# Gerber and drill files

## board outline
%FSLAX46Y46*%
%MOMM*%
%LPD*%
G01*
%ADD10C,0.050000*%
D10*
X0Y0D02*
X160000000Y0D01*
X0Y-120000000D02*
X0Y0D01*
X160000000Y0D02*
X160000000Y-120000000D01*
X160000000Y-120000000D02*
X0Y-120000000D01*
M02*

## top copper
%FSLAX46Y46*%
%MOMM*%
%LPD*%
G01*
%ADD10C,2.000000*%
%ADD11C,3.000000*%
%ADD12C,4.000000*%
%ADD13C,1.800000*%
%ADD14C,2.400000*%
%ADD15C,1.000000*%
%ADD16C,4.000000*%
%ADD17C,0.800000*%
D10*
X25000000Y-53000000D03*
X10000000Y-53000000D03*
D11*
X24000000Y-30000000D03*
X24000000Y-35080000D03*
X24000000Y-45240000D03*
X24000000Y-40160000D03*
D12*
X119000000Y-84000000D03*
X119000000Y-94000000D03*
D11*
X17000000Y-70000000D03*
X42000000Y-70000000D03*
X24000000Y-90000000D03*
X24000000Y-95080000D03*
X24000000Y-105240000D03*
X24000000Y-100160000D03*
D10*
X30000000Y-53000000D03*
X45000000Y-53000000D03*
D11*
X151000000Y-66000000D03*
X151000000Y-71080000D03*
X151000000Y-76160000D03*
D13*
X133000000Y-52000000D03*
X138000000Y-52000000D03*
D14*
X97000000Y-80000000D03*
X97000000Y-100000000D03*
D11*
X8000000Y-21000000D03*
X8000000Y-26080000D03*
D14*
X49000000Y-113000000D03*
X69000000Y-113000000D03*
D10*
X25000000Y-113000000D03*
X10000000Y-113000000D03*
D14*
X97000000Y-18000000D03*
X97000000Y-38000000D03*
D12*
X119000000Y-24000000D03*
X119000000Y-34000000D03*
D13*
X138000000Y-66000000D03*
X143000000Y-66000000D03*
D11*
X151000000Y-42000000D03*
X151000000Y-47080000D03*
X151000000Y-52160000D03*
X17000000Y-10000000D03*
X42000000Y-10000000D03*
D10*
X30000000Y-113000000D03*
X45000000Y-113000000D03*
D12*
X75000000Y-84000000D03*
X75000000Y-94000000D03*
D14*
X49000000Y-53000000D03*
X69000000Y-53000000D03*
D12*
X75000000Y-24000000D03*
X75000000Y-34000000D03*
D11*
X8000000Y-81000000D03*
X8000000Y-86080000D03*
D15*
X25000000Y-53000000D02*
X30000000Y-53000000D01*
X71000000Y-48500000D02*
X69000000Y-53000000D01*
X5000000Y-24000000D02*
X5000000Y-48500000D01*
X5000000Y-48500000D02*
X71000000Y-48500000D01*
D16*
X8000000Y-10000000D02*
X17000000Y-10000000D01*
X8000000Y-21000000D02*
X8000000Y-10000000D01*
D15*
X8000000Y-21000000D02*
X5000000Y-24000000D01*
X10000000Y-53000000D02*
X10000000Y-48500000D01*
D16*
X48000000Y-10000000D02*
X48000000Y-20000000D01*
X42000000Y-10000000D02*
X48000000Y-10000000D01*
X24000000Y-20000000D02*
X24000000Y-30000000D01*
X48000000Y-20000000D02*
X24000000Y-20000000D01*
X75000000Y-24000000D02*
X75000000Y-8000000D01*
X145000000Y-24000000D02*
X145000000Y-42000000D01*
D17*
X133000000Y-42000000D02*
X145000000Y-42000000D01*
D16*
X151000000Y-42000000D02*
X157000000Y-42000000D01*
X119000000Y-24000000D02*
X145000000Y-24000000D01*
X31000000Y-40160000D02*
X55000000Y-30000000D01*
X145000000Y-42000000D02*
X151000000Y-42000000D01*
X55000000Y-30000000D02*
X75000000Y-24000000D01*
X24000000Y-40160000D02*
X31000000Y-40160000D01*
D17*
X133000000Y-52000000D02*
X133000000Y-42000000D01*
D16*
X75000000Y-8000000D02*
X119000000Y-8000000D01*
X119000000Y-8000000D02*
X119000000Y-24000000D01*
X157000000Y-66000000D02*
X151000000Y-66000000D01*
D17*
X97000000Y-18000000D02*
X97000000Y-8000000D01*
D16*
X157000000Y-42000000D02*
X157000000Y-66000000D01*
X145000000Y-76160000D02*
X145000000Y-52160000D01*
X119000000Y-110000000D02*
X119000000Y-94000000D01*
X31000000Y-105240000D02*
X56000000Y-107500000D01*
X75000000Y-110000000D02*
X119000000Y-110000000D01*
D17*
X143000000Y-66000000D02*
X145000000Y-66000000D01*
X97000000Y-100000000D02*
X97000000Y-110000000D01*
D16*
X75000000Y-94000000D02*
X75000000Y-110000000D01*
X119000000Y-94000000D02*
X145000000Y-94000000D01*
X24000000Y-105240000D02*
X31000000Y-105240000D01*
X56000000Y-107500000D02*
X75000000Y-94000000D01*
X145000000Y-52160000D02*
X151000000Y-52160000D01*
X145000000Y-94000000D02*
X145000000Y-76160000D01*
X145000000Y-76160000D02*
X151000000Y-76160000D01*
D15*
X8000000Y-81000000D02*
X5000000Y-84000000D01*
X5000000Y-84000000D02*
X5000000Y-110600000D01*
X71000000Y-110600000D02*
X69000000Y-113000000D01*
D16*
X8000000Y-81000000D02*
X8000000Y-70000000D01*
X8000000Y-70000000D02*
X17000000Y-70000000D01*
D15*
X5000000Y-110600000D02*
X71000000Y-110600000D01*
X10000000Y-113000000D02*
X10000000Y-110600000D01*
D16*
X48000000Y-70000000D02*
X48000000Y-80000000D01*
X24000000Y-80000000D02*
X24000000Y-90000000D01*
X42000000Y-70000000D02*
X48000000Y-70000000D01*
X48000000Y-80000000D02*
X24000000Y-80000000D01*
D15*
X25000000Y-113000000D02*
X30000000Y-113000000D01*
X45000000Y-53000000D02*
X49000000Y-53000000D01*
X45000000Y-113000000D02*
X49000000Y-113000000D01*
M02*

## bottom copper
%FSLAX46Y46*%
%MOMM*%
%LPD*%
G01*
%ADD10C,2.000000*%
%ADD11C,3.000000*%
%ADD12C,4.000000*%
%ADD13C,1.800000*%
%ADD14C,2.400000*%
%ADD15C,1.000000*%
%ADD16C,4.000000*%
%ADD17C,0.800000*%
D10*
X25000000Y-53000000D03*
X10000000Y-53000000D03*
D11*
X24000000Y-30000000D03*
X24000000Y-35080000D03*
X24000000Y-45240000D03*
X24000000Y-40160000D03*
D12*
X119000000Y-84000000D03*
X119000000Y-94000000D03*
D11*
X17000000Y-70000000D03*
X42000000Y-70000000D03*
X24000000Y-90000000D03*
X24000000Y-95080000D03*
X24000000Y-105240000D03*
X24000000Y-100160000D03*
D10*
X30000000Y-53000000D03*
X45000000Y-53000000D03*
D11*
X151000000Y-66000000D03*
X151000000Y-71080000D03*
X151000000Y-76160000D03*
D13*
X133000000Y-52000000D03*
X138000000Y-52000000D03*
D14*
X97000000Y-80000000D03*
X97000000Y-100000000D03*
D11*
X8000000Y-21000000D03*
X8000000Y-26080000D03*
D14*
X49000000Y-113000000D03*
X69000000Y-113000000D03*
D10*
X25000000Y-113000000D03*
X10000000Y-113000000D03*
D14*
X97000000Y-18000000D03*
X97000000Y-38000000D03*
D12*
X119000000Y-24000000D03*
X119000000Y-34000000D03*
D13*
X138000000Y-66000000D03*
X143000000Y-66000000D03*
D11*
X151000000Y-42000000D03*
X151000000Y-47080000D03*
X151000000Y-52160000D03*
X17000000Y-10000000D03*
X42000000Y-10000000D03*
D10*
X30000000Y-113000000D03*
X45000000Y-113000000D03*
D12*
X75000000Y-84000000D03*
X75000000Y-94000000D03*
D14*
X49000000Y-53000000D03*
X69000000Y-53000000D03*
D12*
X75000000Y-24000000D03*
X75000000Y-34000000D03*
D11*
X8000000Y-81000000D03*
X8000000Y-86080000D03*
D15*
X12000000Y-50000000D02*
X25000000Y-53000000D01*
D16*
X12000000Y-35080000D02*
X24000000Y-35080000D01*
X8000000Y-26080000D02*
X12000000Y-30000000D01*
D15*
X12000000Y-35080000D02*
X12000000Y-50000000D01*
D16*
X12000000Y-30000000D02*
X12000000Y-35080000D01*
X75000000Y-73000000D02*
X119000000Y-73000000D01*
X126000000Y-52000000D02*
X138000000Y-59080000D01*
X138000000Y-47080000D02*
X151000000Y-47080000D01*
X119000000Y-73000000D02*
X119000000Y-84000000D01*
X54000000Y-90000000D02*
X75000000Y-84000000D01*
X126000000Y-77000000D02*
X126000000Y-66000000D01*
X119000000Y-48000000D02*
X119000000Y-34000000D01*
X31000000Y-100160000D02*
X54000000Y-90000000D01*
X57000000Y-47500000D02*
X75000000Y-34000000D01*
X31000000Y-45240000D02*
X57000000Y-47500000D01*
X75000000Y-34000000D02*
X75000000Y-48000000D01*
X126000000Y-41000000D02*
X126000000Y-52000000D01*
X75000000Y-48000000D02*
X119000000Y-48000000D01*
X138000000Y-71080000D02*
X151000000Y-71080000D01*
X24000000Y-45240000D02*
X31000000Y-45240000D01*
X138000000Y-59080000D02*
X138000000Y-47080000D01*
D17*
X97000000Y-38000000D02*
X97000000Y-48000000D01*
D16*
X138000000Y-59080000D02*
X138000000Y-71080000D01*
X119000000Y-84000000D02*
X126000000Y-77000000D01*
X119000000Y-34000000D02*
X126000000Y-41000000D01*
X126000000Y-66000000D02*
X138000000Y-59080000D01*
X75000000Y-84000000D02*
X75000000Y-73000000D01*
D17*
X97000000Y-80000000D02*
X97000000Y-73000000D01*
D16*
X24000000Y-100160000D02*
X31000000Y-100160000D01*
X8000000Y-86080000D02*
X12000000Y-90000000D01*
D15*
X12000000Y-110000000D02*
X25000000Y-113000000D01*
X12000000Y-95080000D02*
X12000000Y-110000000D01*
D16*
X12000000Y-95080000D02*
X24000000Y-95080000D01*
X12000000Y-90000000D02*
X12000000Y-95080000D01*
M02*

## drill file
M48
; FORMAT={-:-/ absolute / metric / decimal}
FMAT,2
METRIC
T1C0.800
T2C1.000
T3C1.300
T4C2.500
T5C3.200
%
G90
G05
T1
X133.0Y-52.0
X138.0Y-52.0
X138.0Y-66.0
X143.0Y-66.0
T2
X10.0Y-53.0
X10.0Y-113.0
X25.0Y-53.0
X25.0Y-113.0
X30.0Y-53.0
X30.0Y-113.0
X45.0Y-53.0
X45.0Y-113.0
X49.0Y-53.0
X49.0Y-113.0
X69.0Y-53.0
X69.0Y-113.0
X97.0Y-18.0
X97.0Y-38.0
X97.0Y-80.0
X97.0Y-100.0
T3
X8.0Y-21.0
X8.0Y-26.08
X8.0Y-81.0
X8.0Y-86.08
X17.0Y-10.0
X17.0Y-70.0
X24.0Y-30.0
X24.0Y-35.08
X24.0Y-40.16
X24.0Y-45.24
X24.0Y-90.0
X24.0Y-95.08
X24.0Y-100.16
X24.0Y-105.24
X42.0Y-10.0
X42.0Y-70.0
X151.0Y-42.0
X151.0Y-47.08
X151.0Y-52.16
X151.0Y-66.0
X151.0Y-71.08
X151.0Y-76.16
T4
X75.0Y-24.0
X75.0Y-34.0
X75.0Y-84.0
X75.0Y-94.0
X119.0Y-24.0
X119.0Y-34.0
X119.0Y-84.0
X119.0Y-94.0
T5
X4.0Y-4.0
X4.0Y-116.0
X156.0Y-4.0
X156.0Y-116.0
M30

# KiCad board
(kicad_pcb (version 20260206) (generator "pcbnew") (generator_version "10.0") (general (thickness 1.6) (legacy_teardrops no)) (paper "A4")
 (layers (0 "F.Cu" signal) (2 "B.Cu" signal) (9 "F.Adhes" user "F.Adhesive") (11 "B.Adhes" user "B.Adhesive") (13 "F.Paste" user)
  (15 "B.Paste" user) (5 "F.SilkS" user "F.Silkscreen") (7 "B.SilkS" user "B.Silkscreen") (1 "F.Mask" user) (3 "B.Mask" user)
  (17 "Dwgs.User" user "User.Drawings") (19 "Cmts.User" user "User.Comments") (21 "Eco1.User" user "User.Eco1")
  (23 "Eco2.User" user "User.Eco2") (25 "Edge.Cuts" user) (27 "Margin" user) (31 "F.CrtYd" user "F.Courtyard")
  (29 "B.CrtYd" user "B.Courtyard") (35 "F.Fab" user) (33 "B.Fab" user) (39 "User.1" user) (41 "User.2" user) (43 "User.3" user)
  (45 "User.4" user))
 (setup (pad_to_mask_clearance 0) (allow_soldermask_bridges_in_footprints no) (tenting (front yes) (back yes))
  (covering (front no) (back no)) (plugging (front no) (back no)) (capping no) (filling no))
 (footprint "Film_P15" (layer "F.Cu") (at 25 53 180)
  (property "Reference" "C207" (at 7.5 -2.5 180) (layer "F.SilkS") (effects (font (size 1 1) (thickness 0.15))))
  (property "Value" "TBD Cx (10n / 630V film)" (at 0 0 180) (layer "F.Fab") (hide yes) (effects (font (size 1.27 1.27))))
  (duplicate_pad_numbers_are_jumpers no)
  (pad "1" thru_hole circle (at 0 0 180) (size 2 2) (drill 1) (layers "*.Cu" "*.Mask") (remove_unused_layers no) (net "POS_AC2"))
  (pad "2" thru_hole circle (at 15 0 180) (size 2 2) (drill 1) (layers "*.Cu" "*.Mask") (remove_unused_layers no) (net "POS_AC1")))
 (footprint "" (layer "F.Cu") (at 156 4)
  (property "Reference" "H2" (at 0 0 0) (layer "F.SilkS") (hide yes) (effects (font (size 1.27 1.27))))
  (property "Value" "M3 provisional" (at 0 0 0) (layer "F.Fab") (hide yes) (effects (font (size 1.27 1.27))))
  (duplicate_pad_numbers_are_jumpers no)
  (pad "" np_thru_hole circle (at 0 0) (size 3.2 3.2) (drill 3.2) (layers "*.Cu" "*.Mask")))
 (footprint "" (layer "F.Cu") (at 4 4)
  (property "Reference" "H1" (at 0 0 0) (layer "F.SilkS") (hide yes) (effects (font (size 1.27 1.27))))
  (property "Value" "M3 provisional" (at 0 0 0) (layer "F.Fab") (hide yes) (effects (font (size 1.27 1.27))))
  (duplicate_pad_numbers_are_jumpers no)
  (pad "" np_thru_hole circle (at 0 0) (size 3.2 3.2) (drill 3.2) (layers "*.Cu" "*.Mask")))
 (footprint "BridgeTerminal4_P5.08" (layer "F.Cu") (at 24 30 -90)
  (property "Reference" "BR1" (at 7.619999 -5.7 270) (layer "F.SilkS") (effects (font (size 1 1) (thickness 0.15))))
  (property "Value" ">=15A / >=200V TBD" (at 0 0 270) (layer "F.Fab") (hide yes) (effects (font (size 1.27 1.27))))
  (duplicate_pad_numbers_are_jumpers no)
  (pad "AC1" thru_hole circle (at 0 0 270) (size 3 3) (drill 1.3) (layers "*.Cu" "*.Mask") (remove_unused_layers no) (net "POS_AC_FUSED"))
  (pad "AC2" thru_hole circle (at 5.08 0 270) (size 3 3) (drill 1.3) (layers "*.Cu" "*.Mask") (remove_unused_layers no) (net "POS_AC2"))
  (pad "N" thru_hole circle (at 15.24 0 270) (size 3 3) (drill 1.3) (layers "*.Cu" "*.Mask") (remove_unused_layers no) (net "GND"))
  (pad "P" thru_hole circle (at 10.16 0 270) (size 3 3) (drill 1.3) (layers "*.Cu" "*.Mask") (remove_unused_layers no) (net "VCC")))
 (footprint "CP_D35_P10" (layer "F.Cu") (at 119 84 -90)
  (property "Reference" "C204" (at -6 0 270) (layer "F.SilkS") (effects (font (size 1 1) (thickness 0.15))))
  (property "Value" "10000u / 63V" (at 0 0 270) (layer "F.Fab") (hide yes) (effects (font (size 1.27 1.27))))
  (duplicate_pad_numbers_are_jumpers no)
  (pad "1" thru_hole circle (at 0 0 270) (size 4 4) (drill 2.5) (layers "*.Cu" "*.Mask") (remove_unused_layers no) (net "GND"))
  (pad "2" thru_hole circle (at 10 0 270) (size 4 4) (drill 2.5) (layers "*.Cu" "*.Mask") (remove_unused_layers no) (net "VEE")))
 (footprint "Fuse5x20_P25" (layer "F.Cu") (at 17 70)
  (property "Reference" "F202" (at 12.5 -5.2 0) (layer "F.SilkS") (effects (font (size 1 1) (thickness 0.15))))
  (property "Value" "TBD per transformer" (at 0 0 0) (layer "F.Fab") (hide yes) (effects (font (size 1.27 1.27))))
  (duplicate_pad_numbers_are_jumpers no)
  (pad "1" thru_hole circle (at 0 0) (size 3 3) (drill 1.3) (layers "*.Cu" "*.Mask") (remove_unused_layers no) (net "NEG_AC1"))
  (pad "2" thru_hole circle (at 25 0) (size 3 3) (drill 1.3) (layers "*.Cu" "*.Mask") (remove_unused_layers no) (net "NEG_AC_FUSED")))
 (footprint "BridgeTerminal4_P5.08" (layer "F.Cu") (at 24 90 -90)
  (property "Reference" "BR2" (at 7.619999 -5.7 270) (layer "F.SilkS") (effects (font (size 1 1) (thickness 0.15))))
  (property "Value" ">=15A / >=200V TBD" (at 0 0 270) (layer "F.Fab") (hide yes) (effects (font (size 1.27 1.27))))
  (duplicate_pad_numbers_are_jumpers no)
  (pad "AC1" thru_hole circle (at 0 0 270) (size 3 3) (drill 1.3) (layers "*.Cu" "*.Mask") (remove_unused_layers no) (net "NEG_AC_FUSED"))
  (pad "AC2" thru_hole circle (at 5.08 0 270) (size 3 3) (drill 1.3) (layers "*.Cu" "*.Mask") (remove_unused_layers no) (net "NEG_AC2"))
  (pad "N" thru_hole circle (at 15.24 0 270) (size 3 3) (drill 1.3) (layers "*.Cu" "*.Mask") (remove_unused_layers no) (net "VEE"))
  (pad "P" thru_hole circle (at 10.16 0 270) (size 3 3) (drill 1.3) (layers "*.Cu" "*.Mask") (remove_unused_layers no) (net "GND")))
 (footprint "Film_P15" (layer "F.Cu") (at 30 53)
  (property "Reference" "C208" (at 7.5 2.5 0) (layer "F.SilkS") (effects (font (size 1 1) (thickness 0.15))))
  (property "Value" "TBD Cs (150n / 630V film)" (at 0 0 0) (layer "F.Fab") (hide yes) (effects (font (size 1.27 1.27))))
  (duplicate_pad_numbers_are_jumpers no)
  (pad "1" thru_hole circle (at 0 0) (size 2 2) (drill 1) (layers "*.Cu" "*.Mask") (remove_unused_layers no) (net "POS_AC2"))
  (pad "2" thru_hole circle (at 15 0) (size 2 2) (drill 1) (layers "*.Cu" "*.Mask") (remove_unused_layers no) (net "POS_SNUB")))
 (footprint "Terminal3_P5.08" (layer "F.Cu") (at 151 66 -90)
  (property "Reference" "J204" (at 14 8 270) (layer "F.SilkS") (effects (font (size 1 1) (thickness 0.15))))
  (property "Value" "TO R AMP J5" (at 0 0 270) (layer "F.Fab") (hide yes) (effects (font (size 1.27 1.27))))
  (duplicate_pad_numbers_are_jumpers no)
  (pad "1" thru_hole circle (at 0 0 270) (size 3 3) (drill 1.3) (layers "*.Cu" "*.Mask") (remove_unused_layers no) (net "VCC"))
  (pad "2" thru_hole circle (at 5.08 0 270) (size 3 3) (drill 1.3) (layers "*.Cu" "*.Mask") (remove_unused_layers no) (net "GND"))
  (pad "3" thru_hole circle (at 10.16 0 270) (size 3 3) (drill 1.3) (layers "*.Cu" "*.Mask") (remove_unused_layers no) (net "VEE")))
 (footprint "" (layer "F.Cu") (at 156 116)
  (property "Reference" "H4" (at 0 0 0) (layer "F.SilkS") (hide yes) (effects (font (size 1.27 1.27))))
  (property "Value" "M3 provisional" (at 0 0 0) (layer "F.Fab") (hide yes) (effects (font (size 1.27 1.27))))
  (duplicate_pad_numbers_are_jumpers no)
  (pad "" np_thru_hole circle (at 0 0) (size 3.2 3.2) (drill 3.2) (layers "*.Cu" "*.Mask")))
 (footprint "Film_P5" (layer "F.Cu") (at 133 52)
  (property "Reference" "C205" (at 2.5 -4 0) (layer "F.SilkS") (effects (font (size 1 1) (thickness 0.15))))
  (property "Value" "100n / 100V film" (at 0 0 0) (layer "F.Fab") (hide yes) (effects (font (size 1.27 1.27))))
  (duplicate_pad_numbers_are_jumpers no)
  (pad "1" thru_hole circle (at 0 0) (size 1.8 1.8) (drill 0.8) (layers "*.Cu" "*.Mask") (remove_unused_layers no) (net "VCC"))
  (pad "2" thru_hole circle (at 5 0) (size 1.8 1.8) (drill 0.8) (layers "*.Cu" "*.Mask") (remove_unused_layers no) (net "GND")))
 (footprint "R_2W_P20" (layer "F.Cu") (at 97 80 -90)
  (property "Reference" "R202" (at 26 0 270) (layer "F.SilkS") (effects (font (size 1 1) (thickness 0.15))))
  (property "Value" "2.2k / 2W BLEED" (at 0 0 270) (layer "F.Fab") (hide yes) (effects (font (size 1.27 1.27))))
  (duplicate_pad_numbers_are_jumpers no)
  (pad "1" thru_hole circle (at 0 0 270) (size 2.4 2.4) (drill 1) (layers "*.Cu" "*.Mask") (remove_unused_layers no) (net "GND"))
  (pad "2" thru_hole circle (at 20 0 270) (size 2.4 2.4) (drill 1) (layers "*.Cu" "*.Mask") (remove_unused_layers no) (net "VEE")))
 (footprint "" (layer "F.Cu") (at 4 116)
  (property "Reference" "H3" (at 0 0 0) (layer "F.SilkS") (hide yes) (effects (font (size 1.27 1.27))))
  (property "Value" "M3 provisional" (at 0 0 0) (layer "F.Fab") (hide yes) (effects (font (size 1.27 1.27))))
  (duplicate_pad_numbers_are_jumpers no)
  (pad "" np_thru_hole circle (at 0 0) (size 3.2 3.2) (drill 3.2) (layers "*.Cu" "*.Mask")))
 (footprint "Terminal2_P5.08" (layer "F.Cu") (at 8 21 -90)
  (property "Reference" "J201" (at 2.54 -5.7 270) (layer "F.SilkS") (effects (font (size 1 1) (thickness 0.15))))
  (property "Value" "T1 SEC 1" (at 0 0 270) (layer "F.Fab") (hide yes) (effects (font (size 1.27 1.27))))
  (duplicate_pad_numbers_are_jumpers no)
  (pad "1" thru_hole circle (at 0 0 270) (size 3 3) (drill 1.3) (layers "*.Cu" "*.Mask") (remove_unused_layers no) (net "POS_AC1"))
  (pad "2" thru_hole circle (at 5.08 0 270) (size 3 3) (drill 1.3) (layers "*.Cu" "*.Mask") (remove_unused_layers no) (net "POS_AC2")))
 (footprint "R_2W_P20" (layer "F.Cu") (at 49 113)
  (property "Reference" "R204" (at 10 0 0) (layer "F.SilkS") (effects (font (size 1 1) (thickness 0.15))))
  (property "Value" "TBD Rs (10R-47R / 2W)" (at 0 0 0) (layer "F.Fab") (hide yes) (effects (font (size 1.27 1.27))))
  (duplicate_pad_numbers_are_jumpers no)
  (pad "1" thru_hole circle (at 0 0) (size 2.4 2.4) (drill 1) (layers "*.Cu" "*.Mask") (remove_unused_layers no) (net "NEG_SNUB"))
  (pad "2" thru_hole circle (at 20 0) (size 2.4 2.4) (drill 1) (layers "*.Cu" "*.Mask") (remove_unused_layers no) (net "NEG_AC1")))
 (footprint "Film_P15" (layer "F.Cu") (at 25 113 180)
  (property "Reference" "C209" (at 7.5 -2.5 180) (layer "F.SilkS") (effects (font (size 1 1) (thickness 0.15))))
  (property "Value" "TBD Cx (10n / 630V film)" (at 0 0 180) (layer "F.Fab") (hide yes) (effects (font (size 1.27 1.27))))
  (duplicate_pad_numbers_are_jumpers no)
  (pad "1" thru_hole circle (at 0 0 180) (size 2 2) (drill 1) (layers "*.Cu" "*.Mask") (remove_unused_layers no) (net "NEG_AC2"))
  (pad "2" thru_hole circle (at 15 0 180) (size 2 2) (drill 1) (layers "*.Cu" "*.Mask") (remove_unused_layers no) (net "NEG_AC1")))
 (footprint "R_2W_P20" (layer "F.Cu") (at 97 18 -90)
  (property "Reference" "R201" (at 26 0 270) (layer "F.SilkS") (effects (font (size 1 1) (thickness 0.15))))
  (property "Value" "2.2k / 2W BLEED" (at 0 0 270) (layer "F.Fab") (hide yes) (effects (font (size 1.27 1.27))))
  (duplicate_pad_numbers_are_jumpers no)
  (pad "1" thru_hole circle (at 0 0 270) (size 2.4 2.4) (drill 1) (layers "*.Cu" "*.Mask") (remove_unused_layers no) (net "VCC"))
  (pad "2" thru_hole circle (at 20 0 270) (size 2.4 2.4) (drill 1) (layers "*.Cu" "*.Mask") (remove_unused_layers no) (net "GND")))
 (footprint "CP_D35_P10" (layer "F.Cu") (at 119 24 -90)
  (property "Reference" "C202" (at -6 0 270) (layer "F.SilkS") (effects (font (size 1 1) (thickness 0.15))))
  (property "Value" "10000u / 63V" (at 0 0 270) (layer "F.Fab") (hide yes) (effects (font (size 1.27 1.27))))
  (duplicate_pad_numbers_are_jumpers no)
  (pad "1" thru_hole circle (at 0 0 270) (size 4 4) (drill 2.5) (layers "*.Cu" "*.Mask") (remove_unused_layers no) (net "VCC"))
  (pad "2" thru_hole circle (at 10 0 270) (size 4 4) (drill 2.5) (layers "*.Cu" "*.Mask") (remove_unused_layers no) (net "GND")))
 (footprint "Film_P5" (layer "F.Cu") (at 138 66)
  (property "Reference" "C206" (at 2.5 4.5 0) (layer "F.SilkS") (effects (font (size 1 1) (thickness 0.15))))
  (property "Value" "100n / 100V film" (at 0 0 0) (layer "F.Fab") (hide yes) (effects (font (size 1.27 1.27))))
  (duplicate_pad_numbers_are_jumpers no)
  (pad "1" thru_hole circle (at 0 0) (size 1.8 1.8) (drill 0.8) (layers "*.Cu" "*.Mask") (remove_unused_layers no) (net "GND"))
  (pad "2" thru_hole circle (at 5 0) (size 1.8 1.8) (drill 0.8) (layers "*.Cu" "*.Mask") (remove_unused_layers no) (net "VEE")))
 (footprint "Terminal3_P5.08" (layer "F.Cu") (at 151 42 -90)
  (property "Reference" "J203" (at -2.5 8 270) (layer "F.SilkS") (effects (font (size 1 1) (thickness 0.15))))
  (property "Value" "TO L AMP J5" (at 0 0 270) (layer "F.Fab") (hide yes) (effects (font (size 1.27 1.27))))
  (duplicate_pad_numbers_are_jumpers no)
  (pad "1" thru_hole circle (at 0 0 270) (size 3 3) (drill 1.3) (layers "*.Cu" "*.Mask") (remove_unused_layers no) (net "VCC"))
  (pad "2" thru_hole circle (at 5.08 0 270) (size 3 3) (drill 1.3) (layers "*.Cu" "*.Mask") (remove_unused_layers no) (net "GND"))
  (pad "3" thru_hole circle (at 10.16 0 270) (size 3 3) (drill 1.3) (layers "*.Cu" "*.Mask") (remove_unused_layers no) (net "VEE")))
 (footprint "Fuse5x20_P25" (layer "F.Cu") (at 17 10)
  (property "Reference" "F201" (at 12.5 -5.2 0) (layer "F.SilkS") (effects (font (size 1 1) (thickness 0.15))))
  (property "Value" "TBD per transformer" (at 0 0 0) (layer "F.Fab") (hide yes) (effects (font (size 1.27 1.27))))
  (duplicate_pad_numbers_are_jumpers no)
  (pad "1" thru_hole circle (at 0 0) (size 3 3) (drill 1.3) (layers "*.Cu" "*.Mask") (remove_unused_layers no) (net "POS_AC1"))
  (pad "2" thru_hole circle (at 25 0) (size 3 3) (drill 1.3) (layers "*.Cu" "*.Mask") (remove_unused_layers no) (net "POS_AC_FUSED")))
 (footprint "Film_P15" (layer "F.Cu") (at 30 113)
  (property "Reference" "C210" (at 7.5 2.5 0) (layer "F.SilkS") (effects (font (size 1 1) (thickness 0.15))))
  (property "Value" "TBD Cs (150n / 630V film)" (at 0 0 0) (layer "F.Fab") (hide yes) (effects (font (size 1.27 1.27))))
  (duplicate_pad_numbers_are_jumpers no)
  (pad "1" thru_hole circle (at 0 0) (size 2 2) (drill 1) (layers "*.Cu" "*.Mask") (remove_unused_layers no) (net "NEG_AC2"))
  (pad "2" thru_hole circle (at 15 0) (size 2 2) (drill 1) (layers "*.Cu" "*.Mask") (remove_unused_layers no) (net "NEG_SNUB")))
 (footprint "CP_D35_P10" (layer "F.Cu") (at 75 84 -90)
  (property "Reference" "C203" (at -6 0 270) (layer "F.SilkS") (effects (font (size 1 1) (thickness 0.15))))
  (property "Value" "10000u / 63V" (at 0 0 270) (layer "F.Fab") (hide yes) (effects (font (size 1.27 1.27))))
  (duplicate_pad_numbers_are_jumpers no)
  (pad "1" thru_hole circle (at 0 0 270) (size 4 4) (drill 2.5) (layers "*.Cu" "*.Mask") (remove_unused_layers no) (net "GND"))
  (pad "2" thru_hole circle (at 10 0 270) (size 4 4) (drill 2.5) (layers "*.Cu" "*.Mask") (remove_unused_layers no) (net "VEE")))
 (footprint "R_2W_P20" (layer "F.Cu") (at 49 53)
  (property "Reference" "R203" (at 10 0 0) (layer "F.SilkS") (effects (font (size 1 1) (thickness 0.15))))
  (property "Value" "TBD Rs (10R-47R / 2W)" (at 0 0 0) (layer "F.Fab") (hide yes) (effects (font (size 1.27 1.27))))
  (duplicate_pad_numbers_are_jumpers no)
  (pad "1" thru_hole circle (at 0 0) (size 2.4 2.4) (drill 1) (layers "*.Cu" "*.Mask") (remove_unused_layers no) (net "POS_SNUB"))
  (pad "2" thru_hole circle (at 20 0) (size 2.4 2.4) (drill 1) (layers "*.Cu" "*.Mask") (remove_unused_layers no) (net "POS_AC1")))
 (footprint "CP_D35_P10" (layer "F.Cu") (at 75 24 -90)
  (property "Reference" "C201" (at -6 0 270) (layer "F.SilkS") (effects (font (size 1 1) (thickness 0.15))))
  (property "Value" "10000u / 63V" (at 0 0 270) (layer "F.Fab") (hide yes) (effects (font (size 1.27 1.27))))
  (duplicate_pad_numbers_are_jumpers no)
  (pad "1" thru_hole circle (at 0 0 270) (size 4 4) (drill 2.5) (layers "*.Cu" "*.Mask") (remove_unused_layers no) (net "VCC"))
  (pad "2" thru_hole circle (at 10 0 270) (size 4 4) (drill 2.5) (layers "*.Cu" "*.Mask") (remove_unused_layers no) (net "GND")))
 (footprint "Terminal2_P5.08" (layer "F.Cu") (at 8 81 -90)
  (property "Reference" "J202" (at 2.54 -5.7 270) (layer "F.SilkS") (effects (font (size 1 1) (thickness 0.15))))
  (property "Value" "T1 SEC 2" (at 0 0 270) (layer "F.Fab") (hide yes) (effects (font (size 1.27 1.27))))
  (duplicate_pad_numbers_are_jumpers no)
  (pad "1" thru_hole circle (at 0 0 270) (size 3 3) (drill 1.3) (layers "*.Cu" "*.Mask") (remove_unused_layers no) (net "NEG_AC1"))
  (pad "2" thru_hole circle (at 5.08 0 270) (size 3 3) (drill 1.3) (layers "*.Cu" "*.Mask") (remove_unused_layers no) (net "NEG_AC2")))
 (gr_line (start 0 0) (end 160 0) (stroke (width 0.05) (type default)) (layer "Edge.Cuts"))
 (gr_line (start 0 120) (end 0 0) (stroke (width 0.05) (type default)) (layer "Edge.Cuts"))
 (gr_line (start 160 0) (end 160 120) (stroke (width 0.05) (type default)) (layer "Edge.Cuts"))
 (gr_line (start 160 120) (end 0 120) (stroke (width 0.05) (type default)) (layer "Edge.Cuts"))
 (segment (start 25 53) (end 30 53) (width 1) (layer "F.Cu") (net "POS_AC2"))
 (segment (start 12 50) (end 25 53) (width 1) (layer "B.Cu") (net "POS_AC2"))
 (segment (start 12 35.08) (end 24 35.08) (width 4) (layer "B.Cu") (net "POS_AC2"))
 (segment (start 8 26.08) (end 12 30) (width 4) (layer "B.Cu") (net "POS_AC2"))
 (segment (start 12 35.08) (end 12 50) (width 1) (layer "B.Cu") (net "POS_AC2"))
 (segment (start 12 30) (end 12 35.08) (width 4) (layer "B.Cu") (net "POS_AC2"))
 (segment (start 71 48.5) (end 69 53) (width 1) (layer "F.Cu") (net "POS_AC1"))
 (segment (start 5 24) (end 5 48.5) (width 1) (layer "F.Cu") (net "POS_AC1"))
 (segment (start 5 48.5) (end 71 48.5) (width 1) (layer "F.Cu") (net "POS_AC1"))
 (segment (start 8 10) (end 17 10) (width 4) (layer "F.Cu") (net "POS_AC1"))
 (segment (start 8 21) (end 8 10) (width 4) (layer "F.Cu") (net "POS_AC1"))
 (segment (start 8 21) (end 5 24) (width 1) (layer "F.Cu") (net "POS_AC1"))
 (segment (start 10 53) (end 10 48.5) (width 1) (layer "F.Cu") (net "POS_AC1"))
 (segment (start 48 10) (end 48 20) (width 4) (layer "F.Cu") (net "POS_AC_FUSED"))
 (segment (start 42 10) (end 48 10) (width 4) (layer "F.Cu") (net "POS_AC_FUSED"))
 (segment (start 24 20) (end 24 30) (width 4) (layer "F.Cu") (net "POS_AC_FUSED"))
 (segment (start 48 20) (end 24 20) (width 4) (layer "F.Cu") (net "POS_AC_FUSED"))
 (segment (start 75 73) (end 119 73) (width 4) (layer "B.Cu") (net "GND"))
 (segment (start 126 52) (end 138 59.08) (width 4) (layer "B.Cu") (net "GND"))
 (segment (start 138 47.08) (end 151 47.08) (width 4) (layer "B.Cu") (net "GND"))
 (segment (start 119 73) (end 119 84) (width 4) (layer "B.Cu") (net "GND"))
 (segment (start 54 90) (end 75 84) (width 4) (layer "B.Cu") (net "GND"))
 (segment (start 126 77) (end 126 66) (width 4) (layer "B.Cu") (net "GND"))
 (segment (start 119 48) (end 119 34) (width 4) (layer "B.Cu") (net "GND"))
 (segment (start 31 100.16) (end 54 90) (width 4) (layer "B.Cu") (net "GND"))
 (segment (start 57 47.5) (end 75 34) (width 4) (layer "B.Cu") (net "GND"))
 (segment (start 31 45.24) (end 57 47.5) (width 4) (layer "B.Cu") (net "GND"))
 (segment (start 75 34) (end 75 48) (width 4) (layer "B.Cu") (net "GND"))
 (segment (start 126 41) (end 126 52) (width 4) (layer "B.Cu") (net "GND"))
 (segment (start 75 48) (end 119 48) (width 4) (layer "B.Cu") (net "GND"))
 (segment (start 138 71.08) (end 151 71.08) (width 4) (layer "B.Cu") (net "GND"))
 (segment (start 24 45.24) (end 31 45.24) (width 4) (layer "B.Cu") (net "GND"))
 (segment (start 138 59.08) (end 138 47.08) (width 4) (layer "B.Cu") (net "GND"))
 (segment (start 97 38) (end 97 48) (width 0.8) (layer "B.Cu") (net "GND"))
 (segment (start 138 59.08) (end 138 71.08) (width 4) (layer "B.Cu") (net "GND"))
 (segment (start 119 84) (end 126 77) (width 4) (layer "B.Cu") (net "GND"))
 (segment (start 119 34) (end 126 41) (width 4) (layer "B.Cu") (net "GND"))
 (segment (start 126 66) (end 138 59.08) (width 4) (layer "B.Cu") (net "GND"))
 (segment (start 75 84) (end 75 73) (width 4) (layer "B.Cu") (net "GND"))
 (segment (start 97 80) (end 97 73) (width 0.8) (layer "B.Cu") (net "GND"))
 (segment (start 24 100.16) (end 31 100.16) (width 4) (layer "B.Cu") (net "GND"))
 (segment (start 75 24) (end 75 8) (width 4) (layer "F.Cu") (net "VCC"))
 (segment (start 145 24) (end 145 42) (width 4) (layer "F.Cu") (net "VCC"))
 (segment (start 133 42) (end 145 42) (width 0.8) (layer "F.Cu") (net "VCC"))
 (segment (start 151 42) (end 157 42) (width 4) (layer "F.Cu") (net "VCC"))
 (segment (start 119 24) (end 145 24) (width 4) (layer "F.Cu") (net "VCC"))
 (segment (start 31 40.16) (end 55 30) (width 4) (layer "F.Cu") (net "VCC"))
 (segment (start 145 42) (end 151 42) (width 4) (layer "F.Cu") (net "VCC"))
 (segment (start 55 30) (end 75 24) (width 4) (layer "F.Cu") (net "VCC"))
 (segment (start 24 40.16) (end 31 40.16) (width 4) (layer "F.Cu") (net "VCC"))
 (segment (start 133 52) (end 133 42) (width 0.8) (layer "F.Cu") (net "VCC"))
 (segment (start 75 8) (end 119 8) (width 4) (layer "F.Cu") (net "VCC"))
 (segment (start 119 8) (end 119 24) (width 4) (layer "F.Cu") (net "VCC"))
 (segment (start 157 66) (end 151 66) (width 4) (layer "F.Cu") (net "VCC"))
 (segment (start 97 18) (end 97 8) (width 0.8) (layer "F.Cu") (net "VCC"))
 (segment (start 157 42) (end 157 66) (width 4) (layer "F.Cu") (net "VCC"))
 (segment (start 145 76.16) (end 145 52.16) (width 4) (layer "F.Cu") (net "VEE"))
 (segment (start 119 110) (end 119 94) (width 4) (layer "F.Cu") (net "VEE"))
 (segment (start 31 105.24) (end 56 107.5) (width 4) (layer "F.Cu") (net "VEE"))
 (segment (start 75 110) (end 119 110) (width 4) (layer "F.Cu") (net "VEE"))
 (segment (start 143 66) (end 145 66) (width 0.8) (layer "F.Cu") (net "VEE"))
 (segment (start 97 100) (end 97 110) (width 0.8) (layer "F.Cu") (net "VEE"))
 (segment (start 75 94) (end 75 110) (width 4) (layer "F.Cu") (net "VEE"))
 (segment (start 119 94) (end 145 94) (width 4) (layer "F.Cu") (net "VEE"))
 (segment (start 24 105.24) (end 31 105.24) (width 4) (layer "F.Cu") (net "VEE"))
 (segment (start 56 107.5) (end 75 94) (width 4) (layer "F.Cu") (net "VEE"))
 (segment (start 145 52.16) (end 151 52.16) (width 4) (layer "F.Cu") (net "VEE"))
 (segment (start 145 94) (end 145 76.16) (width 4) (layer "F.Cu") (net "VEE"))
 (segment (start 145 76.16) (end 151 76.16) (width 4) (layer "F.Cu") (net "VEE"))
 (segment (start 8 81) (end 5 84) (width 1) (layer "F.Cu") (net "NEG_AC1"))
 (segment (start 5 84) (end 5 110.6) (width 1) (layer "F.Cu") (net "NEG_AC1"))
 (segment (start 71 110.6) (end 69 113) (width 1) (layer "F.Cu") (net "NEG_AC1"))
 (segment (start 8 81) (end 8 70) (width 4) (layer "F.Cu") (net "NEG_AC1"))
 (segment (start 8 70) (end 17 70) (width 4) (layer "F.Cu") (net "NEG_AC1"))
 (segment (start 5 110.6) (end 71 110.6) (width 1) (layer "F.Cu") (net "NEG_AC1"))
 (segment (start 10 113) (end 10 110.6) (width 1) (layer "F.Cu") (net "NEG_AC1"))
 (segment (start 48 70) (end 48 80) (width 4) (layer "F.Cu") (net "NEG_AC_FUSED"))
 (segment (start 24 80) (end 24 90) (width 4) (layer "F.Cu") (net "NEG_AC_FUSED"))
 (segment (start 42 70) (end 48 70) (width 4) (layer "F.Cu") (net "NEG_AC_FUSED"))
 (segment (start 48 80) (end 24 80) (width 4) (layer "F.Cu") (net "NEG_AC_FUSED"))
 (segment (start 25 113) (end 30 113) (width 1) (layer "F.Cu") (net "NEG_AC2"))
 (segment (start 8 86.08) (end 12 90) (width 4) (layer "B.Cu") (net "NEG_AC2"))
 (segment (start 12 110) (end 25 113) (width 1) (layer "B.Cu") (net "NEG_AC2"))
 (segment (start 12 95.08) (end 12 110) (width 1) (layer "B.Cu") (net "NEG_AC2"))
 (segment (start 12 95.08) (end 24 95.08) (width 4) (layer "B.Cu") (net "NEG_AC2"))
 (segment (start 12 90) (end 12 95.08) (width 4) (layer "B.Cu") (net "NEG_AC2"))
 (segment (start 45 53) (end 49 53) (width 1) (layer "F.Cu") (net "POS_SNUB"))
 (segment (start 45 113) (end 49 113) (width 1) (layer "F.Cu") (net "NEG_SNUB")))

